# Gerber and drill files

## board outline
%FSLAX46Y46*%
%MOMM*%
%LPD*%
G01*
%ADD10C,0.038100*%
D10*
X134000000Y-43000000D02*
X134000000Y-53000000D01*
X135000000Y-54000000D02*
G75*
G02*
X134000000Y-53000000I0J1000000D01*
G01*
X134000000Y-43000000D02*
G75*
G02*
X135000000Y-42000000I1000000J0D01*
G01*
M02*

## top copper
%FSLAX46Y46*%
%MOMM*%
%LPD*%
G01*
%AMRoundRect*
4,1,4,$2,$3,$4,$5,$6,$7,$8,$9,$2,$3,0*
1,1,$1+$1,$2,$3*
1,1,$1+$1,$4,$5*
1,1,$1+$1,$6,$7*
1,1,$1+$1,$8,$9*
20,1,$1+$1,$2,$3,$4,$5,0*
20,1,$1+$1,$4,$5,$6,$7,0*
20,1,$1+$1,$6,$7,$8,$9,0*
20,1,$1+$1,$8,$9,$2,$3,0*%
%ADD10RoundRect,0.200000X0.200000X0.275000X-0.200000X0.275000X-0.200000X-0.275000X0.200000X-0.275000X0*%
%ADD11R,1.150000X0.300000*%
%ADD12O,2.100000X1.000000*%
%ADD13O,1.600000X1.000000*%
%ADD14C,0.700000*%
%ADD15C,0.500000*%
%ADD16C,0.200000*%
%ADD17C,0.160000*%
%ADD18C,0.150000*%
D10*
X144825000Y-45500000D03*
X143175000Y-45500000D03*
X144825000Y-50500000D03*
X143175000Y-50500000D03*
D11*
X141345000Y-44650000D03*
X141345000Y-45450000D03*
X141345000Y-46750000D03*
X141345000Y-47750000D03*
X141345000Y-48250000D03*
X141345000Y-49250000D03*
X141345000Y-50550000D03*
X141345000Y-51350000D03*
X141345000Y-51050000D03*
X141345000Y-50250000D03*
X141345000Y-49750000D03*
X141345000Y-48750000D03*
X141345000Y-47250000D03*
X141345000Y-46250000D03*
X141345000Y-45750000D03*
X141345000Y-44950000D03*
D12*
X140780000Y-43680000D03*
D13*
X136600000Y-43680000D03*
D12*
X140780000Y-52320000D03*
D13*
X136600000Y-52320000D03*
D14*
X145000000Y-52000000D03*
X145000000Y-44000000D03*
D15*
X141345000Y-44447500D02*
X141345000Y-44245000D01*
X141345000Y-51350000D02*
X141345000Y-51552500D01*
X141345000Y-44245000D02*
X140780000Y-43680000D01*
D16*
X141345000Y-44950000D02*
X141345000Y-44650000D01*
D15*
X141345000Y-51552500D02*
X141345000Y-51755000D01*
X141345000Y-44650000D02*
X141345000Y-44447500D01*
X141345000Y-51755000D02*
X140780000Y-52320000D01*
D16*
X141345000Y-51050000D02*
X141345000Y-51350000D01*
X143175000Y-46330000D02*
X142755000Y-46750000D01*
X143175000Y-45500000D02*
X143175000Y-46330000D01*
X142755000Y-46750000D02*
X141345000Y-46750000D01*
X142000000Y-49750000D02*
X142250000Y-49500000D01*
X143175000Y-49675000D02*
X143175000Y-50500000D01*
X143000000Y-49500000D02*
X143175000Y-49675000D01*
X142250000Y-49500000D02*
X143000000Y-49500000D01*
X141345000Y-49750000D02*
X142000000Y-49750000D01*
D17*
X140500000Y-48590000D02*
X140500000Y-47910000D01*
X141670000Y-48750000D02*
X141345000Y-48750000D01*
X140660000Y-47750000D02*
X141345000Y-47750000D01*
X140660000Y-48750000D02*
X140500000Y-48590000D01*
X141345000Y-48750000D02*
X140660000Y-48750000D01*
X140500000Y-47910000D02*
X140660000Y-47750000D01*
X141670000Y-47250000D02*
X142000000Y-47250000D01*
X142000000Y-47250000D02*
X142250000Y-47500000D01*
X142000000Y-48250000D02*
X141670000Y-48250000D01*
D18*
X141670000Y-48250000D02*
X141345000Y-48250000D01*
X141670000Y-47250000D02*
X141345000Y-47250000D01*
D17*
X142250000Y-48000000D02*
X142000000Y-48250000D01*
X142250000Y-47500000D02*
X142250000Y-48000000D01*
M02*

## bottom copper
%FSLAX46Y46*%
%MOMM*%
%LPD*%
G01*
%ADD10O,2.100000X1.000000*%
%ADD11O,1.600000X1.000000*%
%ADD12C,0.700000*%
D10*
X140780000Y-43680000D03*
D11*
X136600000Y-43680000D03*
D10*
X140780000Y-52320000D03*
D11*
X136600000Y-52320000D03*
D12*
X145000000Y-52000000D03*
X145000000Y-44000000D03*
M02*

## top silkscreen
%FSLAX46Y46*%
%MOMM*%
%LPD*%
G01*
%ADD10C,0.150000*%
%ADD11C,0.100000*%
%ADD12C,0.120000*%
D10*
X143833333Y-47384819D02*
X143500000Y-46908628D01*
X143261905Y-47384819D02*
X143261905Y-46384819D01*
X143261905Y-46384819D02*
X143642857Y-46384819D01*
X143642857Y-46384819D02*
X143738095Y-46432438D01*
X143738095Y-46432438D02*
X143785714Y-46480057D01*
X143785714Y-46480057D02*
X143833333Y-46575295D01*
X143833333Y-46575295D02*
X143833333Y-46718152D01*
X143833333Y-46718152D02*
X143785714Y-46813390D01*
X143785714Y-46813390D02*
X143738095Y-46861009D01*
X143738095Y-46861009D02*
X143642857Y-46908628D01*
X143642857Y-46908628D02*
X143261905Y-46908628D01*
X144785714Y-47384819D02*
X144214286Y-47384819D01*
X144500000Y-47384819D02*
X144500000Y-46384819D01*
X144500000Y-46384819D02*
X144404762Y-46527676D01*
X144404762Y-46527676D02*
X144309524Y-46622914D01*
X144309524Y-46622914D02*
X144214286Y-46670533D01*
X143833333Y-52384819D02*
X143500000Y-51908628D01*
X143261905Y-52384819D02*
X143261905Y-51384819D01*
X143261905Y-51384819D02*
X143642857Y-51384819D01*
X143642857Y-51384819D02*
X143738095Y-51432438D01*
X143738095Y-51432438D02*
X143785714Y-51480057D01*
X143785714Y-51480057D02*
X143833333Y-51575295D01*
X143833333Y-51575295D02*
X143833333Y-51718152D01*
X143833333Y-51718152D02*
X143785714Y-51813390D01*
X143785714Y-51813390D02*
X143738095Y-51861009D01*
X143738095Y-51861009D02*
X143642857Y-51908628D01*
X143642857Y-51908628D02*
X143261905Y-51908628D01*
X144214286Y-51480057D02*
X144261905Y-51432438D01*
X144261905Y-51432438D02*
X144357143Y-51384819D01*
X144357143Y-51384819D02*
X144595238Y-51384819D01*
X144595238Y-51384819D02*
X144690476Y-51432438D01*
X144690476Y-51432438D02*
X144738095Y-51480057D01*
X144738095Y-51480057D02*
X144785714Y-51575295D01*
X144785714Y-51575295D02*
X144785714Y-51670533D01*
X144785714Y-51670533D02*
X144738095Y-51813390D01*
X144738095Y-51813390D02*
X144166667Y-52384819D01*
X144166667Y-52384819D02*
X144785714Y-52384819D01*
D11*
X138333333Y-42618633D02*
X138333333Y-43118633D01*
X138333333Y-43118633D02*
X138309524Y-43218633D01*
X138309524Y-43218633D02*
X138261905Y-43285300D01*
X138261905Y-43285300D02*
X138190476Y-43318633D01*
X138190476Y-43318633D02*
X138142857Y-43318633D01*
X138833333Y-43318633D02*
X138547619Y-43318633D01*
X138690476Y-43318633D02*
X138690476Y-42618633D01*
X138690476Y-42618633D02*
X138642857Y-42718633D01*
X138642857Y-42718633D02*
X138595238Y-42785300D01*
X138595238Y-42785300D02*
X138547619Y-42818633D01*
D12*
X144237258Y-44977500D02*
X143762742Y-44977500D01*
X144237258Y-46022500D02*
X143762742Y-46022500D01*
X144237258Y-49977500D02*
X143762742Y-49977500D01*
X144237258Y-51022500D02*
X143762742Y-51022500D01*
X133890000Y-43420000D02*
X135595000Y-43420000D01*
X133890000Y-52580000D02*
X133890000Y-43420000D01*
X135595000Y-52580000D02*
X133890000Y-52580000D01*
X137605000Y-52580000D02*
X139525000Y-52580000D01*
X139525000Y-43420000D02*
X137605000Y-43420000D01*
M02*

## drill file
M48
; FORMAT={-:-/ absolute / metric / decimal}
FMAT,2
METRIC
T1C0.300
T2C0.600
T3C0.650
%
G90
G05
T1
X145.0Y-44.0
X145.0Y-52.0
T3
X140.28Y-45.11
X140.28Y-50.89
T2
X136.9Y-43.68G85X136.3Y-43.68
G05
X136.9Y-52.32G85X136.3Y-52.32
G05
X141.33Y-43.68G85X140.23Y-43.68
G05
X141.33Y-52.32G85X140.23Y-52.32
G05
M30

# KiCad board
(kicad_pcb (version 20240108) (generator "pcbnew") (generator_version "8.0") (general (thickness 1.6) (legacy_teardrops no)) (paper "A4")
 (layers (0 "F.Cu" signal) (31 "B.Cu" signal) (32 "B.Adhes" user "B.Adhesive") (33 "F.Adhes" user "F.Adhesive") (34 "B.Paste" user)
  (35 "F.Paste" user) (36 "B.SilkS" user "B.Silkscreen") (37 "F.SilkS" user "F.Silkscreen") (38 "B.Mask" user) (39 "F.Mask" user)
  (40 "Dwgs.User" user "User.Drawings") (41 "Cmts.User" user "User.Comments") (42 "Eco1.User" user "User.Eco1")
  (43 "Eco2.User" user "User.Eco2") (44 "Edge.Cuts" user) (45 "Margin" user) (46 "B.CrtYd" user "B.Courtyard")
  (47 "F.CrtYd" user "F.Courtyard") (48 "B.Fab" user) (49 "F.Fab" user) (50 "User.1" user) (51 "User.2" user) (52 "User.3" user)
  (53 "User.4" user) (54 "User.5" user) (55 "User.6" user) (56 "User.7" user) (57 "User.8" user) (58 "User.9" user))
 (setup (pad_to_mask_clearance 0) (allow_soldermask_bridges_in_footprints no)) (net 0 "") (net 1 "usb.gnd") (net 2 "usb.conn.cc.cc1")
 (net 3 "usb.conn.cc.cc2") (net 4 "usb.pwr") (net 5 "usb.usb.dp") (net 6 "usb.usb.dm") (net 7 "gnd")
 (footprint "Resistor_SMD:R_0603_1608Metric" (layer "F.Cu") (at 144 45.5 180)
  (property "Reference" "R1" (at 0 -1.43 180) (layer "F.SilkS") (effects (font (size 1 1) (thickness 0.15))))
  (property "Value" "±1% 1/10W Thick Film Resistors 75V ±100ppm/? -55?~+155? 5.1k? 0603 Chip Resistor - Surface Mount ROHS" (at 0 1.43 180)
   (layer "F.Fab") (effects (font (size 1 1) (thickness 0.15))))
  (fp_line (start -0.237258 0.5225) (end 0.237258 0.5225) (stroke (width 0.12) (type solid)) (layer "F.SilkS"))
  (fp_line (start -0.237258 -0.5225) (end 0.237258 -0.5225) (stroke (width 0.12) (type solid)) (layer "F.SilkS"))
  (pad "1" smd roundrect (at -0.825 0 180) (size 0.8 0.95) (layers "F.Cu" "F.Paste" "F.Mask") (roundrect_rratio 0.25) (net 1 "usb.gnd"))
  (pad "2" smd roundrect (at 0.825 0 180) (size 0.8 0.95) (layers "F.Cu" "F.Paste" "F.Mask") (roundrect_rratio 0.25)
   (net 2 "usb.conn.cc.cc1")))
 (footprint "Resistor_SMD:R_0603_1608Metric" (layer "F.Cu") (at 144 50.5 180)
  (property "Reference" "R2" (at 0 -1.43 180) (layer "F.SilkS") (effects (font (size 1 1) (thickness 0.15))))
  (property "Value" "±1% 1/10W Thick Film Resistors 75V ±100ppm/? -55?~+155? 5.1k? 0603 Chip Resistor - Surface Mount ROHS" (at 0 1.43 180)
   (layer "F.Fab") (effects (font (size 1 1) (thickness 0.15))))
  (fp_line (start -0.237258 0.5225) (end 0.237258 0.5225) (stroke (width 0.12) (type solid)) (layer "F.SilkS"))
  (fp_line (start -0.237258 -0.5225) (end 0.237258 -0.5225) (stroke (width 0.12) (type solid)) (layer "F.SilkS"))
  (pad "1" smd roundrect (at -0.825 0 180) (size 0.8 0.95) (layers "F.Cu" "F.Paste" "F.Mask") (roundrect_rratio 0.25) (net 1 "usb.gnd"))
  (pad "2" smd roundrect (at 0.825 0 180) (size 0.8 0.95) (layers "F.Cu" "F.Paste" "F.Mask") (roundrect_rratio 0.25)
   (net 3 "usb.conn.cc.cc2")))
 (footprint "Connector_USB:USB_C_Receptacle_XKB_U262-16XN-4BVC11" (layer "F.Cu") (at 137.675 48 -90)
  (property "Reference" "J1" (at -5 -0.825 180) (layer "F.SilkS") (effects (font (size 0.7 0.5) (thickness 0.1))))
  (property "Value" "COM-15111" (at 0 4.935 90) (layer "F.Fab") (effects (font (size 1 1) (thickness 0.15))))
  (fp_line (start -4.58 3.785) (end -4.58 2.08) (stroke (width 0.12) (type solid)) (layer "F.SilkS"))
  (fp_line (start 4.58 3.785) (end -4.58 3.785) (stroke (width 0.12) (type solid)) (layer "F.SilkS"))
  (fp_line (start 4.58 2.08) (end 4.58 3.785) (stroke (width 0.12) (type solid)) (layer "F.SilkS"))
  (fp_line (start 4.58 0.07) (end 4.58 -1.85) (stroke (width 0.12) (type solid)) (layer "F.SilkS"))
  (fp_line (start -4.58 -1.85) (end -4.58 0.07) (stroke (width 0.12) (type solid)) (layer "F.SilkS"))
  (pad "" np_thru_hole circle (at -2.89 -2.605 270) (size 0.65 0.65) (drill 0.65) (layers "*.Cu" "*.Mask"))
  (pad "" np_thru_hole circle (at 2.89 -2.605 270) (size 0.65 0.65) (drill 0.65) (layers "*.Cu" "*.Mask"))
  (pad "A1" smd rect (at -3.35 -3.67 270) (size 0.3 1.15) (layers "F.Cu" "F.Paste" "F.Mask") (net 1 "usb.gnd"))
  (pad "A4" smd rect (at -2.55 -3.67 270) (size 0.3 1.15) (layers "F.Cu" "F.Paste" "F.Mask") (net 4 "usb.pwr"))
  (pad "A5" smd rect (at -1.25 -3.67 270) (size 0.3 1.15) (layers "F.Cu" "F.Paste" "F.Mask") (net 2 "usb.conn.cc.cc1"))
  (pad "A6" smd rect (at -0.25 -3.67 270) (size 0.3 1.15) (layers "F.Cu" "F.Paste" "F.Mask") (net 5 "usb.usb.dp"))
  (pad "A7" smd rect (at 0.25 -3.67 270) (size 0.3 1.15) (layers "F.Cu" "F.Paste" "F.Mask") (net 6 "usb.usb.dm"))
  (pad "A8" smd rect (at 1.25 -3.67 270) (size 0.3 1.15) (layers "F.Cu" "F.Paste" "F.Mask"))
  (pad "A9" smd rect (at 2.55 -3.67 270) (size 0.3 1.15) (layers "F.Cu" "F.Paste" "F.Mask") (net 4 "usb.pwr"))
  (pad "A12" smd rect (at 3.35 -3.67 270) (size 0.3 1.15) (layers "F.Cu" "F.Paste" "F.Mask") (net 1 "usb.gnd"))
  (pad "B1" smd rect (at 3.05 -3.67 270) (size 0.3 1.15) (layers "F.Cu" "F.Paste" "F.Mask") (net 1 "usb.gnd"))
  (pad "B4" smd rect (at 2.25 -3.67 270) (size 0.3 1.15) (layers "F.Cu" "F.Paste" "F.Mask") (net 4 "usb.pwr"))
  (pad "B5" smd rect (at 1.75 -3.67 270) (size 0.3 1.15) (layers "F.Cu" "F.Paste" "F.Mask") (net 3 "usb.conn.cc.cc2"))
  (pad "B6" smd rect (at 0.75 -3.67 270) (size 0.3 1.15) (layers "F.Cu" "F.Paste" "F.Mask") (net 5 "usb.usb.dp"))
  (pad "B7" smd rect (at -0.75 -3.67 270) (size 0.3 1.15) (layers "F.Cu" "F.Paste" "F.Mask") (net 6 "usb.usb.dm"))
  (pad "B8" smd rect (at -1.75 -3.67 270) (size 0.3 1.15) (layers "F.Cu" "F.Paste" "F.Mask"))
  (pad "B9" smd rect (at -2.25 -3.67 270) (size 0.3 1.15) (layers "F.Cu" "F.Paste" "F.Mask") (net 4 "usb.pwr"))
  (pad "B12" smd rect (at -3.05 -3.67 270) (size 0.3 1.15) (layers "F.Cu" "F.Paste" "F.Mask") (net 1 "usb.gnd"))
  (pad "S1" thru_hole oval (at -4.32 -3.105 270) (size 1 2.1) (drill oval 0.6 1.7) (layers "*.Cu" "*.Mask") (remove_unused_layers no)
   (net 1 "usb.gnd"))
  (pad "S1" thru_hole oval (at -4.32 1.075 270) (size 1 1.6) (drill oval 0.6 1.2) (layers "*.Cu" "*.Mask") (remove_unused_layers no)
   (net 1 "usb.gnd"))
  (pad "S1" thru_hole oval (at 4.32 -3.105 270) (size 1 2.1) (drill oval 0.6 1.7) (layers "*.Cu" "*.Mask") (remove_unused_layers no)
   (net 1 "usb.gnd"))
  (pad "S1" thru_hole oval (at 4.32 1.075 270) (size 1 1.6) (drill oval 0.6 1.2) (layers "*.Cu" "*.Mask") (remove_unused_layers no)
   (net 1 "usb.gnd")))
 (gr_line (start 134 43) (end 134 53) (stroke (width 0.0381) (type solid)) (layer "Edge.Cuts"))
 (gr_arc (start 135 54) (mid 134.292893 53.707107) (end 134 53) (stroke (width 0.0381) (type solid)) (layer "Edge.Cuts"))
 (gr_arc (start 134 43) (mid 134.292893 42.292893) (end 135 42) (stroke (width 0.0381) (type solid)) (layer "Edge.Cuts"))
 (via (at 145 52) (size 0.7) (drill 0.3) (layers "F.Cu" "B.Cu") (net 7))
 (via (at 145 44) (size 0.7) (drill 0.3) (layers "F.Cu" "B.Cu") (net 7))
 (segment (start 141.345 44.4475) (end 141.345 44.245) (width 0.5) (layer "F.Cu") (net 1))
 (segment (start 141.345 51.35) (end 141.345 51.5525) (width 0.5) (layer "F.Cu") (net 1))
 (segment (start 141.345 44.245) (end 140.78 43.68) (width 0.5) (layer "F.Cu") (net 1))
 (segment (start 141.345 44.95) (end 141.345 44.65) (width 0.2) (layer "F.Cu") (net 1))
 (segment (start 141.345 51.5525) (end 141.345 51.755) (width 0.5) (layer "F.Cu") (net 1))
 (segment (start 141.345 44.65) (end 141.345 44.4475) (width 0.5) (layer "F.Cu") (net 1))
 (segment (start 141.345 51.755) (end 140.78 52.32) (width 0.5) (layer "F.Cu") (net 1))
 (segment (start 141.345 51.05) (end 141.345 51.35) (width 0.2) (layer "F.Cu") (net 1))
 (segment (start 143.175 46.33) (end 142.755 46.75) (width 0.2) (layer "F.Cu") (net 2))
 (segment (start 143.175 45.5) (end 143.175 46.33) (width 0.2) (layer "F.Cu") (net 2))
 (segment (start 142.755 46.75) (end 141.345 46.75) (width 0.2) (layer "F.Cu") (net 2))
 (segment (start 142 49.75) (end 142.25 49.5) (width 0.2) (layer "F.Cu") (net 3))
 (segment (start 143.175 49.675) (end 143.175 50.5) (width 0.2) (layer "F.Cu") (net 3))
 (segment (start 143 49.5) (end 143.175 49.675) (width 0.2) (layer "F.Cu") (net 3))
 (segment (start 142.25 49.5) (end 143 49.5) (width 0.2) (layer "F.Cu") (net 3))
 (segment (start 141.345 49.75) (end 142 49.75) (width 0.2) (layer "F.Cu") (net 3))
 (segment (start 140.5 48.59) (end 140.5 47.91) (width 0.16) (layer "F.Cu") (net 5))
 (segment (start 141.67 48.75) (end 141.345 48.75) (width 0.16) (layer "F.Cu") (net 5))
 (segment (start 140.66 47.75) (end 141.345 47.75) (width 0.16) (layer "F.Cu") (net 5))
 (segment (start 140.66 48.75) (end 140.5 48.59) (width 0.16) (layer "F.Cu") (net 5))
 (segment (start 141.345 48.75) (end 140.66 48.75) (width 0.16) (layer "F.Cu") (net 5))
 (segment (start 140.5 47.91) (end 140.66 47.75) (width 0.16) (layer "F.Cu") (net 5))
 (segment (start 141.67 47.25) (end 142 47.25) (width 0.16) (layer "F.Cu") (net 6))
 (segment (start 142 47.25) (end 142.25 47.5) (width 0.16) (layer "F.Cu") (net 6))
 (segment (start 142 48.25) (end 141.67 48.25) (width 0.16) (layer "F.Cu") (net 6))
 (segment (start 141.67 48.25) (end 141.345 48.25) (width 0.15) (layer "F.Cu") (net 6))
 (segment (start 141.67 47.25) (end 141.345 47.25) (width 0.15) (layer "F.Cu") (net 6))
 (segment (start 142.25 48) (end 142 48.25) (width 0.16) (layer "F.Cu") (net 6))
 (segment (start 142.25 47.5) (end 142.25 48) (width 0.16) (layer "F.Cu") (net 6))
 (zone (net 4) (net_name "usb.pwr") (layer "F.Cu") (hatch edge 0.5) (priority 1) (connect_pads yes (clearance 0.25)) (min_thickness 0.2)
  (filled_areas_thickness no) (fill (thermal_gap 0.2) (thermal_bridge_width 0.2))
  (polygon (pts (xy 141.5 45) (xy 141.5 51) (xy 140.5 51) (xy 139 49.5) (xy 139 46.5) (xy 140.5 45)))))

